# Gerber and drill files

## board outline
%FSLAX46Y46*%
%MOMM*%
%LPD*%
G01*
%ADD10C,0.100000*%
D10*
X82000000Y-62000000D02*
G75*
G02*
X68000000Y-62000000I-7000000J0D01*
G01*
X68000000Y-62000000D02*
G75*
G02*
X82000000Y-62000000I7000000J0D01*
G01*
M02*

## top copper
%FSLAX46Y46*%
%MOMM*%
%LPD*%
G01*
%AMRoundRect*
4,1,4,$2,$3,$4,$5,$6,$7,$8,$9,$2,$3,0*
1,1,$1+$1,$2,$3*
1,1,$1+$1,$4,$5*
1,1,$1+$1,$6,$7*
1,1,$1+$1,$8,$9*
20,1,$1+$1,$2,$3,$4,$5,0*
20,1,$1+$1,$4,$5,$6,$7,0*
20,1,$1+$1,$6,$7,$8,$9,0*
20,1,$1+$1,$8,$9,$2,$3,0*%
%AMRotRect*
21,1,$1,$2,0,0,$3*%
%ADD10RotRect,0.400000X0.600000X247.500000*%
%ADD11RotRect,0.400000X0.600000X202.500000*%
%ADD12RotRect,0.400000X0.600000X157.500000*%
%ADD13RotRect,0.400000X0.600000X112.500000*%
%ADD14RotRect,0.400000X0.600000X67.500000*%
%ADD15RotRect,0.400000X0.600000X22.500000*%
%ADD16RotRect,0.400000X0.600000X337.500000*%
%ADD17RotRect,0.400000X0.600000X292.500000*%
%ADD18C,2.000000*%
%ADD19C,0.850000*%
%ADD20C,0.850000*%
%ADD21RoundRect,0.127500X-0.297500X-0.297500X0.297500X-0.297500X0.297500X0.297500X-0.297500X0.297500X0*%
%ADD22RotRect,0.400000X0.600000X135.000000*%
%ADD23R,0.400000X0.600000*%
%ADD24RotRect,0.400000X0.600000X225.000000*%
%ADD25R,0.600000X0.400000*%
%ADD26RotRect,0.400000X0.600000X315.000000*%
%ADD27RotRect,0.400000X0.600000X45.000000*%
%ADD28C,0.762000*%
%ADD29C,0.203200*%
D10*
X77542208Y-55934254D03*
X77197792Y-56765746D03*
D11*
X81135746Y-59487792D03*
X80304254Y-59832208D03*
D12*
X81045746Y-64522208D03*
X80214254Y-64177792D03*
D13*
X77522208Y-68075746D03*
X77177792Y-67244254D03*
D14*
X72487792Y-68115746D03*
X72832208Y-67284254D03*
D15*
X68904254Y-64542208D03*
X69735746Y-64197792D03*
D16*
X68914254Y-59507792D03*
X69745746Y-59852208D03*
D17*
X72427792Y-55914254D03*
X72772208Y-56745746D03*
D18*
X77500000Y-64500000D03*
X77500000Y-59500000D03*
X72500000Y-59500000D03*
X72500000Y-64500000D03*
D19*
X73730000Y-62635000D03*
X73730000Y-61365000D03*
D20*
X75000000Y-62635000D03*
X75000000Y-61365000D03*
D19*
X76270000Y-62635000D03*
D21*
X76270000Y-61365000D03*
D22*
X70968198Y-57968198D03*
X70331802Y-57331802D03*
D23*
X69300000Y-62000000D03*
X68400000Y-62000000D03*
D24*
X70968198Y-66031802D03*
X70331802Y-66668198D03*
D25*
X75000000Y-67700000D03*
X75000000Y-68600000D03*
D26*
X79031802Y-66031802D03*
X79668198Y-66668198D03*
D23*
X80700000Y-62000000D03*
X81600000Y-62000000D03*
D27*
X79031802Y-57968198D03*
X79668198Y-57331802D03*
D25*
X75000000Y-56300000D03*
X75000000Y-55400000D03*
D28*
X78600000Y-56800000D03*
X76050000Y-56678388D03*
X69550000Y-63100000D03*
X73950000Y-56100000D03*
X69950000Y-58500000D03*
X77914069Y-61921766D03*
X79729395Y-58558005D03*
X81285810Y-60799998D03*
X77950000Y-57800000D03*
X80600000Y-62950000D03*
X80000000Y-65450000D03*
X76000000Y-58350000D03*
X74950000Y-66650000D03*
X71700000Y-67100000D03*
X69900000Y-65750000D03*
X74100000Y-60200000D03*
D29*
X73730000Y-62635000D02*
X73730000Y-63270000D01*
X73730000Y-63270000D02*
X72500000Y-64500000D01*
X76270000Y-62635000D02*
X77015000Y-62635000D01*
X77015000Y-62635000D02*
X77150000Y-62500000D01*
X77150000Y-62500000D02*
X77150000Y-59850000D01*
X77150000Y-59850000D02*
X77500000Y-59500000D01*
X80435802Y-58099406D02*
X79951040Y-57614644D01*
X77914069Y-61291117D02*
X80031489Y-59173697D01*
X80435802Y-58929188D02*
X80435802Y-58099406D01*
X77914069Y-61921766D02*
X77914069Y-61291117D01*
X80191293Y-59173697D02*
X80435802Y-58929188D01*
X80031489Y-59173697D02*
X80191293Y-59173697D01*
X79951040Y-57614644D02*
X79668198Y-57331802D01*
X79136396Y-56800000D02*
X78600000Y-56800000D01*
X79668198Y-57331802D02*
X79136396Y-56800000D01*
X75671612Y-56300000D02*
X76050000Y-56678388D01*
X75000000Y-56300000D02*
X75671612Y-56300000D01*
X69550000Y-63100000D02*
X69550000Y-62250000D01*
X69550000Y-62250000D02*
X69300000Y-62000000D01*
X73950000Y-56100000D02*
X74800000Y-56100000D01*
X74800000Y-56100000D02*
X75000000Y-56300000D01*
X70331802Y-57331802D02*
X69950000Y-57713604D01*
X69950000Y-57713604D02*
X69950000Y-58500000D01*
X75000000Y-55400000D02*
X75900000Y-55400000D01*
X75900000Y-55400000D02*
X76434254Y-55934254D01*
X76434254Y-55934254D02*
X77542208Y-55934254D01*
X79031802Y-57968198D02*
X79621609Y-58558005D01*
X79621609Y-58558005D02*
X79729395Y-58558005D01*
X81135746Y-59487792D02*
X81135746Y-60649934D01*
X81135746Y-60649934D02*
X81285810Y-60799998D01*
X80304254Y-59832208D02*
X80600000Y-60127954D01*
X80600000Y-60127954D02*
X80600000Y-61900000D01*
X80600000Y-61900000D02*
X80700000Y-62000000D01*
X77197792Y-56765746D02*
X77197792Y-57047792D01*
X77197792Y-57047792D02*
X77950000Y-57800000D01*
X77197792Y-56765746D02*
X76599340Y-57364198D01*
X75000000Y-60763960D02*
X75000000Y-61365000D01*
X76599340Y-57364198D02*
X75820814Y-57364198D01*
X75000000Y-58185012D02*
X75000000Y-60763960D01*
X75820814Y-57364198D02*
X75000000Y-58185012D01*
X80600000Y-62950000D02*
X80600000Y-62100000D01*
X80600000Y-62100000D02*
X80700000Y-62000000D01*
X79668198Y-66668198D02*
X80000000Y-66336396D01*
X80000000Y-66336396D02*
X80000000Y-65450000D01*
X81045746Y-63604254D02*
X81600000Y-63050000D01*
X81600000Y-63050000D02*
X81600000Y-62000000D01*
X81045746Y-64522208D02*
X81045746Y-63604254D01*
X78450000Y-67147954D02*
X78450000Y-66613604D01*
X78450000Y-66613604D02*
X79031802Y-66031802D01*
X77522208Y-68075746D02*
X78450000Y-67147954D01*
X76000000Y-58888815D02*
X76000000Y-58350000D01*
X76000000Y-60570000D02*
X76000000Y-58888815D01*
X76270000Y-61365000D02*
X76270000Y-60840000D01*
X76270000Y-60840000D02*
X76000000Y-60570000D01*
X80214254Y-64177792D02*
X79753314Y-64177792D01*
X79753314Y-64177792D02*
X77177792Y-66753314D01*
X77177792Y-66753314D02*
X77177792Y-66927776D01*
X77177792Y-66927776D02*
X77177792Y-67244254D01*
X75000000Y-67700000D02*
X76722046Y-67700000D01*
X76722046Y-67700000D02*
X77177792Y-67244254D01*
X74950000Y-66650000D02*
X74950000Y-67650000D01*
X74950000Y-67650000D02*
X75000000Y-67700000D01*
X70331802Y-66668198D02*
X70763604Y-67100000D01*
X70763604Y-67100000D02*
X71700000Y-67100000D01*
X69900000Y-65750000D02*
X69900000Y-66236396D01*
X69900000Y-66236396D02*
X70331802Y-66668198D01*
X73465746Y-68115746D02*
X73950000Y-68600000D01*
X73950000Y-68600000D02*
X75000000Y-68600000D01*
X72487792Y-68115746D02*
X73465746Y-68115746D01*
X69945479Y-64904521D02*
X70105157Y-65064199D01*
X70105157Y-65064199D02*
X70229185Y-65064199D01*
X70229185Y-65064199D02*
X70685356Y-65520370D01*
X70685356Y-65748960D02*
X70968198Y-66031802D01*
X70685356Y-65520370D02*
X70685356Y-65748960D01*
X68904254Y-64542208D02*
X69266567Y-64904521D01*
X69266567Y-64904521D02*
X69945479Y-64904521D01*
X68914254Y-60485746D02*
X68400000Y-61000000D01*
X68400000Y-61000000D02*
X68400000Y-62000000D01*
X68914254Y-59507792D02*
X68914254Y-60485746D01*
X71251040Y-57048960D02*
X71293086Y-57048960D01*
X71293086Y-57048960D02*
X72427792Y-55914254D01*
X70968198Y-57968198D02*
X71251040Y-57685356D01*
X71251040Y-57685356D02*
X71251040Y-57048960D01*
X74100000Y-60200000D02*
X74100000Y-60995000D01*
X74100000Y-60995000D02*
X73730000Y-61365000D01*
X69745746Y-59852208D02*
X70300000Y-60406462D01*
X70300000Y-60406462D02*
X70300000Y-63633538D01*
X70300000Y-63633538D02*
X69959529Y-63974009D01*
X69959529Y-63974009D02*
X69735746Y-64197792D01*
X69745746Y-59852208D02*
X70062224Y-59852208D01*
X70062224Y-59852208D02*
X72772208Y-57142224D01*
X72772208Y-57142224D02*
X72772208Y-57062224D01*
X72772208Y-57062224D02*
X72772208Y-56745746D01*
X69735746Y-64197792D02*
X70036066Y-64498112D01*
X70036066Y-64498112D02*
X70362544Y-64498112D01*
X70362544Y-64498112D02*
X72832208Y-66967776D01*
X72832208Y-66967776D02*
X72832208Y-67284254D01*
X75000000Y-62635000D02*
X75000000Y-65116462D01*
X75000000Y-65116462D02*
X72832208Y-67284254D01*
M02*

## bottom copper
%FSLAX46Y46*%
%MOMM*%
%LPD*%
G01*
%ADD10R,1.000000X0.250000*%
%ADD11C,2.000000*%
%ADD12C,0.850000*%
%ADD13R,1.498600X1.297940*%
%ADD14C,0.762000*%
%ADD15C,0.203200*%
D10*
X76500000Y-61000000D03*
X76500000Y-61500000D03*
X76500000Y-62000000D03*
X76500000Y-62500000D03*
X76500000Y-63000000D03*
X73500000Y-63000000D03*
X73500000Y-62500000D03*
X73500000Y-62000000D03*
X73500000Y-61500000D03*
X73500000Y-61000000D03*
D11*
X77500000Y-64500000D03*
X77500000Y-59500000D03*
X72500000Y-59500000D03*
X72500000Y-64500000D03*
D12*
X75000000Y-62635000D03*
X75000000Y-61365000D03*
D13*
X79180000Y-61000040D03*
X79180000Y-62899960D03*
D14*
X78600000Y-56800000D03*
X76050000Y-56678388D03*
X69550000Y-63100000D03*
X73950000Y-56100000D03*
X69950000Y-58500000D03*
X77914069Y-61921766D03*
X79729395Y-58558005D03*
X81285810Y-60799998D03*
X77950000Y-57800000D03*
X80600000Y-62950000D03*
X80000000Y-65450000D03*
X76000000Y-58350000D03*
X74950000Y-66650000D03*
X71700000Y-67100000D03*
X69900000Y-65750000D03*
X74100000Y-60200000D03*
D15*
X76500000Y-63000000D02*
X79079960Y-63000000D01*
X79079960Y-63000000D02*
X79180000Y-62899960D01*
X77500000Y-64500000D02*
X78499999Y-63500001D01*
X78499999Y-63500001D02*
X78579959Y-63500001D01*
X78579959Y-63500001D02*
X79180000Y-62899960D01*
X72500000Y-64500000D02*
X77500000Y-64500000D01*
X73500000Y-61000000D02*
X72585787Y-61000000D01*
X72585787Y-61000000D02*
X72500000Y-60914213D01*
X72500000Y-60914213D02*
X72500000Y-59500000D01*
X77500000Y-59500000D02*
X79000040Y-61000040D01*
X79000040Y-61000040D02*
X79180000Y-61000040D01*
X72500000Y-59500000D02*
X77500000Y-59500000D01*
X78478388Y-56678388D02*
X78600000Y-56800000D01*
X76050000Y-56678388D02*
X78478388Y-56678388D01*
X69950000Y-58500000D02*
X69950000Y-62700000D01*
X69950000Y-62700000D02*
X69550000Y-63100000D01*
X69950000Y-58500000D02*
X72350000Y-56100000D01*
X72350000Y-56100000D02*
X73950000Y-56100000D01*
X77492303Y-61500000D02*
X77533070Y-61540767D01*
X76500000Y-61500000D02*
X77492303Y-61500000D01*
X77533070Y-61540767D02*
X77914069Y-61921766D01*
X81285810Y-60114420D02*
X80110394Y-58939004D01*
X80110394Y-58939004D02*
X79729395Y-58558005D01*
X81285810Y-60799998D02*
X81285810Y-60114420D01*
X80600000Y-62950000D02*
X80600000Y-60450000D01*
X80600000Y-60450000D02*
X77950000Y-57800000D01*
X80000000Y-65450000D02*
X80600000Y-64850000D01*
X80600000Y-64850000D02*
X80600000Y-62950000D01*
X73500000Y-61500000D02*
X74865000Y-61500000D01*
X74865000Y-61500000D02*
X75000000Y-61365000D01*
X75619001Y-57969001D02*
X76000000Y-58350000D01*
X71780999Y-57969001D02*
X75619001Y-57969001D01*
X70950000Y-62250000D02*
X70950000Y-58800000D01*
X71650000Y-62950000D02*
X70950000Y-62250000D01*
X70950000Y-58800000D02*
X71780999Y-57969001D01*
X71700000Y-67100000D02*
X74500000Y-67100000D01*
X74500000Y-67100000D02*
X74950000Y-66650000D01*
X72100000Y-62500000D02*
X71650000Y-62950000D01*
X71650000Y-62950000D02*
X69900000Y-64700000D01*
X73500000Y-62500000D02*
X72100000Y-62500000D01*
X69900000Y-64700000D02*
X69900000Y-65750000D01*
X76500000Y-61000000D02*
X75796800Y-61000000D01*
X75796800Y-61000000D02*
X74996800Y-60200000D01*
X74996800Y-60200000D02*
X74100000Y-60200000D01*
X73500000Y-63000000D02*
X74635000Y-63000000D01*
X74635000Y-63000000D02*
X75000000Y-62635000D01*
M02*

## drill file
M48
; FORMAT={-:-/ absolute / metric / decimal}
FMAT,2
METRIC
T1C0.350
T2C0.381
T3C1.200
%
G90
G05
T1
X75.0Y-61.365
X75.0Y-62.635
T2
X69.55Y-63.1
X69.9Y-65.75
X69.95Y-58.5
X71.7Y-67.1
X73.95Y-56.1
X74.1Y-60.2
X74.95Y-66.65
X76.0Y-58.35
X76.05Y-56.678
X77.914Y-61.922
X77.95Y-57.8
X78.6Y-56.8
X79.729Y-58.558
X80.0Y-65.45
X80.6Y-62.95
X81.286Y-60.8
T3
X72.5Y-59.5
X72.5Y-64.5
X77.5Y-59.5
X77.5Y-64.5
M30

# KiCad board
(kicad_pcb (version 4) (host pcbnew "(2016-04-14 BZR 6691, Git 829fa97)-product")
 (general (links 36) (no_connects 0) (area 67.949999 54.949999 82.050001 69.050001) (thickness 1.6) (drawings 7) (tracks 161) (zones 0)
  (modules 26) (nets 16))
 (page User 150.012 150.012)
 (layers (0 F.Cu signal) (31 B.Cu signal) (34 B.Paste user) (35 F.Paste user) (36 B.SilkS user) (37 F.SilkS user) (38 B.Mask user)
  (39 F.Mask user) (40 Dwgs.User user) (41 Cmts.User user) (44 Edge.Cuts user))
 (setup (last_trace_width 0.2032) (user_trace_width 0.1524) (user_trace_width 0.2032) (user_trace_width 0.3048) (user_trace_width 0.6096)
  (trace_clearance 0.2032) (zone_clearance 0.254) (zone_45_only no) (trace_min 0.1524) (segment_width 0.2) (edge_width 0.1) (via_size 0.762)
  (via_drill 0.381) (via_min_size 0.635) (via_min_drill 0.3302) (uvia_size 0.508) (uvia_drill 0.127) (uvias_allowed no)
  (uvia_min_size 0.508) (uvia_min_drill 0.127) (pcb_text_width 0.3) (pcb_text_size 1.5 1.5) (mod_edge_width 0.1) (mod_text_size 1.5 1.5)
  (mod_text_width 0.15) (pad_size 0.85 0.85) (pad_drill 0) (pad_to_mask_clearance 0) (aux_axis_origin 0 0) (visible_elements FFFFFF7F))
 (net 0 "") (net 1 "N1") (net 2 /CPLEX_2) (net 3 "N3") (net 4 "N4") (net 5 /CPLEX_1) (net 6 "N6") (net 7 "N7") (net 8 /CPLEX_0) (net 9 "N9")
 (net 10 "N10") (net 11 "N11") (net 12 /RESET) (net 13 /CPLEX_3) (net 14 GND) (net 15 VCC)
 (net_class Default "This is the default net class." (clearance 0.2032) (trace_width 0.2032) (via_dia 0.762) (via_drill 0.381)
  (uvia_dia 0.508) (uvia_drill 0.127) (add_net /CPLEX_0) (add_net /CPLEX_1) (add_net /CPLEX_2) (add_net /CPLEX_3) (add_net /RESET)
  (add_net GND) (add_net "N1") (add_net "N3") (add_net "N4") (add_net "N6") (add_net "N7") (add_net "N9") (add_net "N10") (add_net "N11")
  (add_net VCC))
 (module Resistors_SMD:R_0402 (layer F.Cu) (at 77.37 56.35 247.5)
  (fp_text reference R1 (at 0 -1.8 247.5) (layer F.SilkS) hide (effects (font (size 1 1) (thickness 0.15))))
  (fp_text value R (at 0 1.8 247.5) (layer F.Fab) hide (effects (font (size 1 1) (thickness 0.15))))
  (pad 1 smd rect (at -0.45 0 247.5) (size 0.4 0.6) (layers F.Cu F.Paste F.Mask) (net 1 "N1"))
  (pad 2 smd rect (at 0.45 0 247.5) (size 0.4 0.6) (layers F.Cu F.Paste F.Mask) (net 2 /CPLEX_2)))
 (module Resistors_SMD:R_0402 (layer F.Cu) (at 80.72 59.66 202.5)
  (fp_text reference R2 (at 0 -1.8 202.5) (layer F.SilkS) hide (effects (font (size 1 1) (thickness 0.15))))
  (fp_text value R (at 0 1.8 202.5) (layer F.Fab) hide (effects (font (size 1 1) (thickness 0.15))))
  (pad 1 smd rect (at -0.45 0 202.5) (size 0.4 0.6) (layers F.Cu F.Paste F.Mask) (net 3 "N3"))
  (pad 2 smd rect (at 0.45 0 202.5) (size 0.4 0.6) (layers F.Cu F.Paste F.Mask) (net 2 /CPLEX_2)))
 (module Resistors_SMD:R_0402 (layer F.Cu) (at 80.63 64.35 157.5)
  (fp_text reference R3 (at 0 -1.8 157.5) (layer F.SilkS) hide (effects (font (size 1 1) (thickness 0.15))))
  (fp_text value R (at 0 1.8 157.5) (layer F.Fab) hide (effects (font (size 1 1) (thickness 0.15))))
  (pad 1 smd rect (at -0.45 0 157.5) (size 0.4 0.6) (layers F.Cu F.Paste F.Mask) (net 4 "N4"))
  (pad 2 smd rect (at 0.45 0 157.5) (size 0.4 0.6) (layers F.Cu F.Paste F.Mask) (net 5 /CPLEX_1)))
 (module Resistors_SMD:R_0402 (layer F.Cu) (at 77.35 67.66 112.5)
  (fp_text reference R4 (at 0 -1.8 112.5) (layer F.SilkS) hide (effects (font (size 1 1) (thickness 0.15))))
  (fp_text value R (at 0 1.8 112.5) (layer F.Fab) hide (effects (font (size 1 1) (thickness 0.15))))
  (pad 1 smd rect (at -0.45 0 112.5) (size 0.4 0.6) (layers F.Cu F.Paste F.Mask) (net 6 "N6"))
  (pad 2 smd rect (at 0.45 0 112.5) (size 0.4 0.6) (layers F.Cu F.Paste F.Mask) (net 5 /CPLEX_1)))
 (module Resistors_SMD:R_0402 (layer F.Cu) (at 72.66 67.7 67.5)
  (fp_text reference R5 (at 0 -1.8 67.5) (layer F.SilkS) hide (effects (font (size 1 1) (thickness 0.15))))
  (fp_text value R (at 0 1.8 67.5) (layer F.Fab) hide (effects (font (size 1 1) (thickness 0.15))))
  (pad 1 smd rect (at -0.45 0 67.5) (size 0.4 0.6) (layers F.Cu F.Paste F.Mask) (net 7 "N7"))
  (pad 2 smd rect (at 0.45 0 67.5) (size 0.4 0.6) (layers F.Cu F.Paste F.Mask) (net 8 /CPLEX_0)))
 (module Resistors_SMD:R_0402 (layer F.Cu) (at 69.32 64.37 22.5)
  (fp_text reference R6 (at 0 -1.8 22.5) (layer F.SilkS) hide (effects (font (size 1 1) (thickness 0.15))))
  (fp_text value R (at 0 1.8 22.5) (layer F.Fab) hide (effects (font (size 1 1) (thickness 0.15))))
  (pad 1 smd rect (at -0.45 0 22.5) (size 0.4 0.6) (layers F.Cu F.Paste F.Mask) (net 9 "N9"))
  (pad 2 smd rect (at 0.45 0 22.5) (size 0.4 0.6) (layers F.Cu F.Paste F.Mask) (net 8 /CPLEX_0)))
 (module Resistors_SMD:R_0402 (layer F.Cu) (at 69.33 59.68 337.5)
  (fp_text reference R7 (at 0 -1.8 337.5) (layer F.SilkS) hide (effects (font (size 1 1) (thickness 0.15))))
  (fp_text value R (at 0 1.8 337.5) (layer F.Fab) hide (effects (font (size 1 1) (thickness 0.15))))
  (pad 1 smd rect (at -0.45 0 337.5) (size 0.4 0.6) (layers F.Cu F.Paste F.Mask) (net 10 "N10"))
  (pad 2 smd rect (at 0.45 0 337.5) (size 0.4 0.6) (layers F.Cu F.Paste F.Mask) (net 8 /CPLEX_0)))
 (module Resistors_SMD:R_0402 (layer F.Cu) (at 72.6 56.33 292.5)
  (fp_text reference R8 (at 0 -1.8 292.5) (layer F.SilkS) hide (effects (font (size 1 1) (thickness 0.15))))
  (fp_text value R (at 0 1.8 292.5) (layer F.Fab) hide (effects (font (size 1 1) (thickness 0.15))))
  (pad 1 smd rect (at -0.45 0 292.5) (size 0.4 0.6) (layers F.Cu F.Paste F.Mask) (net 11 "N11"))
  (pad 2 smd rect (at 0.45 0 292.5) (size 0.4 0.6) (layers F.Cu F.Paste F.Mask) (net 8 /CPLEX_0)))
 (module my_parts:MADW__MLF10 (layer B.Cu) (at 75 62 180)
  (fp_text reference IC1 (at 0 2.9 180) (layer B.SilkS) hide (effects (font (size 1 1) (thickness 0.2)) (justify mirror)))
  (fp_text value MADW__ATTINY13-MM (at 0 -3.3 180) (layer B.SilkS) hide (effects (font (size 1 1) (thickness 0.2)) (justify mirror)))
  (pad 1 smd rect (at -1.5 1 180) (size 1 0.25) (layers B.Cu B.Paste B.Mask) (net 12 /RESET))
  (pad 2 smd rect (at -1.5 0.5 180) (size 1 0.25) (layers B.Cu B.Paste B.Mask) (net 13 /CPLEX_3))
  (pad 3 smd rect (at -1.5 0 180) (size 1 0.25) (layers B.Cu B.Paste B.Mask))
  (pad 4 smd rect (at -1.5 -0.5 180) (size 1 0.25) (layers B.Cu B.Paste B.Mask))
  (pad 5 smd rect (at -1.5 -1 180) (size 1 0.25) (layers B.Cu B.Paste B.Mask) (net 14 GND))
  (pad 6 smd rect (at 1.5 -1 180) (size 1 0.25) (layers B.Cu B.Paste B.Mask) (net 8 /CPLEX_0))
  (pad 7 smd rect (at 1.5 -0.5 180) (size 1 0.25) (layers B.Cu B.Paste B.Mask) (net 5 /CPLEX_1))
  (pad 8 smd rect (at 1.5 0 180) (size 1 0.25) (layers B.Cu B.Paste B.Mask))
  (pad 9 smd rect (at 1.5 0.5 180) (size 1 0.25) (layers B.Cu B.Paste B.Mask) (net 2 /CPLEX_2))
  (pad 10 smd rect (at 1.5 1 180) (size 1 0.25) (layers B.Cu B.Paste B.Mask) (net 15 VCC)))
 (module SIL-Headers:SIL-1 (layer F.Cu) (at 77.5 64.5)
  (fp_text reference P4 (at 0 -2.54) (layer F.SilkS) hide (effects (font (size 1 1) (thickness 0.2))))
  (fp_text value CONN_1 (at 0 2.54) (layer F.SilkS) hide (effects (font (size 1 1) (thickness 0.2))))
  (pad 1 thru_hole circle (at 0 0) (size 2 2) (drill 1.2) (layers *.Cu *.Mask) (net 14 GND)))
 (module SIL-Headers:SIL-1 (layer F.Cu) (at 77.5 59.5)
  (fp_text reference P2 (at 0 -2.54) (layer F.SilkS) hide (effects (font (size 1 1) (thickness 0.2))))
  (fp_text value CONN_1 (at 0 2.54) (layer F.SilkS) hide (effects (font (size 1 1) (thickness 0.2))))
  (pad 1 thru_hole circle (at 0 0) (size 2 2) (drill 1.2) (layers *.Cu *.Mask) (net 15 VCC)))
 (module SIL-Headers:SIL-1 (layer F.Cu) (at 72.5 59.5)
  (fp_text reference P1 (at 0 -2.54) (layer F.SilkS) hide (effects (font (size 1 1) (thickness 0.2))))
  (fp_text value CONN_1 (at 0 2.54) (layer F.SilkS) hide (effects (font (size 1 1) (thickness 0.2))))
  (pad 1 thru_hole circle (at 0 0) (size 2 2) (drill 1.2) (layers *.Cu *.Mask) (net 15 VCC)))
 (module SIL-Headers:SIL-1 (layer F.Cu) (at 72.5 64.5)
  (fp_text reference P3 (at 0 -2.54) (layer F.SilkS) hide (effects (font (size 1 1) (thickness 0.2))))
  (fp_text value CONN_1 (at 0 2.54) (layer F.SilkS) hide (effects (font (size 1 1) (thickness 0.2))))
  (pad 1 thru_hole circle (at 0 0) (size 2 2) (drill 1.2) (layers *.Cu *.Mask) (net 14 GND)))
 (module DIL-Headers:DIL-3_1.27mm (layer F.Cu) (at 75 62) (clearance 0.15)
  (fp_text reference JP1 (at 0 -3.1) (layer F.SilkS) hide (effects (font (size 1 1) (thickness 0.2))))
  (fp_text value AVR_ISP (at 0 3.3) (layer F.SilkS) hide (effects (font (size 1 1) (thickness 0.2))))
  (pad 6 smd circle (at -1.27 0.635) (size 0.85 0.85) (layers F.Cu F.Mask) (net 14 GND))
  (pad 5 smd circle (at -1.27 -0.635) (size 0.85 0.85) (layers F.Cu F.Mask) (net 12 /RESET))
  (pad 4 thru_hole circle (at 0 0.635) (size 0.85 0.85) (drill 0.35) (layers *.Cu F.Mask) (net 8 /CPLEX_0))
  (pad 3 thru_hole circle (at 0 -0.635) (size 0.85 0.85) (drill 0.35) (layers *.Cu F.Mask) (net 2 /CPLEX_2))
  (pad 2 smd circle (at 1.27 0.635) (size 0.85 0.85) (layers F.Cu F.Mask) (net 15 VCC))
  (pad 1 smd roundrect (at 1.27 -0.635) (size 0.85 0.85) (layers F.Cu F.Mask) (roundrect_rratio 0.15) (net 5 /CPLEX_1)))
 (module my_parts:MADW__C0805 (layer B.Cu) (at 79.18 61.95 270)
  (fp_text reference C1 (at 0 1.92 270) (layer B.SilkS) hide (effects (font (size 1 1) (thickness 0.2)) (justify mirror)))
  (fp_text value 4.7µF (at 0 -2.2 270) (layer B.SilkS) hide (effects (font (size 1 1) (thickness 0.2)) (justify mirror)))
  (pad 1 smd rect (at -0.94996 0 270) (size 1.29794 1.4986) (layers B.Cu B.Paste B.Mask) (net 15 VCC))
  (pad 2 smd rect (at 0.94996 0 270) (size 1.29794 1.4986) (layers B.Cu B.Paste B.Mask) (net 14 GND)))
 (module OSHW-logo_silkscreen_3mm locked (layer B.Cu) (at 75 56.8)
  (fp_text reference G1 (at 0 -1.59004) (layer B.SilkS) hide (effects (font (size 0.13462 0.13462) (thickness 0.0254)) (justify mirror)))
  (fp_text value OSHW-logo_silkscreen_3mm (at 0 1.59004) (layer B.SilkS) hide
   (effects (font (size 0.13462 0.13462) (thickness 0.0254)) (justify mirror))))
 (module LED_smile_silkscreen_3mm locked (layer B.Cu) (at 75 67.2)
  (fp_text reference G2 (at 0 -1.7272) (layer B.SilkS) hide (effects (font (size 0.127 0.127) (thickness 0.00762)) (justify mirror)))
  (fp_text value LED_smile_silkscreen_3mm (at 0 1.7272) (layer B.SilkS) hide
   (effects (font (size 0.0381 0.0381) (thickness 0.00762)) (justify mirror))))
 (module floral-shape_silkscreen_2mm (layer F.Cu) (at 75.03 57.9 45)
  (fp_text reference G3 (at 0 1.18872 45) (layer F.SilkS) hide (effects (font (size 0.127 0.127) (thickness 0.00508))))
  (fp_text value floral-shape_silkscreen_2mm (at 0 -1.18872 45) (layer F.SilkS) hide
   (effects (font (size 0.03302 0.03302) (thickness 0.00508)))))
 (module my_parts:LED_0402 (layer F.Cu) (at 70.65 57.65 135)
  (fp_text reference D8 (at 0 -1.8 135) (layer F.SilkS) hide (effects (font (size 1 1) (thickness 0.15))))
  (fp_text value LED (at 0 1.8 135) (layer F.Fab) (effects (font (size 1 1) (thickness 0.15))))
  (pad 1 smd rect (at -0.45 0 135) (size 0.4 0.6) (layers F.Cu F.Paste F.Mask) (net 11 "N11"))
  (pad 2 smd rect (at 0.45 0 135) (size 0.4 0.6) (layers F.Cu F.Paste F.Mask) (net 13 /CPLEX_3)))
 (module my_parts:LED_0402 (layer F.Cu) (at 68.85 62 180)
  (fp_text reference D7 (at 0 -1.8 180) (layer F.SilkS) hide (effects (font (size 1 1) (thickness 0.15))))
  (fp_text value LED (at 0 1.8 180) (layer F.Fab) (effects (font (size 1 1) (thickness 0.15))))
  (pad 1 smd rect (at -0.45 0 180) (size 0.4 0.6) (layers F.Cu F.Paste F.Mask) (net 13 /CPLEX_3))
  (pad 2 smd rect (at 0.45 0 180) (size 0.4 0.6) (layers F.Cu F.Paste F.Mask) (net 10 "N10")))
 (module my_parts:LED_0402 (layer F.Cu) (at 70.65 66.35 225)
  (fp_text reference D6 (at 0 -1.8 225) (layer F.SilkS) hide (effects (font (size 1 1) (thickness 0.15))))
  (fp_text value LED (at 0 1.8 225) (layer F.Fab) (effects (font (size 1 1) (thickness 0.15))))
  (pad 1 smd rect (at -0.45 0 225) (size 0.4 0.6) (layers F.Cu F.Paste F.Mask) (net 9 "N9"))
  (pad 2 smd rect (at 0.45 0 225) (size 0.4 0.6) (layers F.Cu F.Paste F.Mask) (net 5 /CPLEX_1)))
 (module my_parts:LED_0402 (layer F.Cu) (at 75 68.15 270)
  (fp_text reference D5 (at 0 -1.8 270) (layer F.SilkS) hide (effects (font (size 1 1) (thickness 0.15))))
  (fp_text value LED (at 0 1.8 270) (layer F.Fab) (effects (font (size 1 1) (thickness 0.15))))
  (pad 1 smd rect (at -0.45 0 270) (size 0.4 0.6) (layers F.Cu F.Paste F.Mask) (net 5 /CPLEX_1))
  (pad 2 smd rect (at 0.45 0 270) (size 0.4 0.6) (layers F.Cu F.Paste F.Mask) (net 7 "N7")))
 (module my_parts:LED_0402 (layer F.Cu) (at 79.35 66.35 315)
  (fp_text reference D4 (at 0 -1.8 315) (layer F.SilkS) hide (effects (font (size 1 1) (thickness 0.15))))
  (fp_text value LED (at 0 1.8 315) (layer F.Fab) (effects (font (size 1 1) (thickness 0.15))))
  (pad 1 smd rect (at -0.45 0 315) (size 0.4 0.6) (layers F.Cu F.Paste F.Mask) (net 6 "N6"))
  (pad 2 smd rect (at 0.45 0 315) (size 0.4 0.6) (layers F.Cu F.Paste F.Mask) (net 2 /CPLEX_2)))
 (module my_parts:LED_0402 (layer F.Cu) (at 81.15 62)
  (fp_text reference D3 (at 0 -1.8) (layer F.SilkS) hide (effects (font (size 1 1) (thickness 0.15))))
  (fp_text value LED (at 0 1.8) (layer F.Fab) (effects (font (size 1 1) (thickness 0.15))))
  (pad 1 smd rect (at -0.45 0) (size 0.4 0.6) (layers F.Cu F.Paste F.Mask) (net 2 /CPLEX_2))
  (pad 2 smd rect (at 0.45 0) (size 0.4 0.6) (layers F.Cu F.Paste F.Mask) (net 4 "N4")))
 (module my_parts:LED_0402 (layer F.Cu) (at 79.35 57.65 45)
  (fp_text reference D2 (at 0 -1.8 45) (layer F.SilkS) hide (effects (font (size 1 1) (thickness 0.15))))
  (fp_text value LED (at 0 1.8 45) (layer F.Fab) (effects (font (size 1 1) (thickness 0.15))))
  (pad 1 smd rect (at -0.45 0 45) (size 0.4 0.6) (layers F.Cu F.Paste F.Mask) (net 3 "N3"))
  (pad 2 smd rect (at 0.45 0 45) (size 0.4 0.6) (layers F.Cu F.Paste F.Mask) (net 13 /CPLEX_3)))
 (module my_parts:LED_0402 (layer F.Cu) (at 75 55.85 90)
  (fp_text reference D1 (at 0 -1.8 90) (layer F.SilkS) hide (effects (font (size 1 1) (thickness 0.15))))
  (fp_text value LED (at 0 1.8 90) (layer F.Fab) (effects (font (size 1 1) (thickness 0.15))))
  (pad 1 smd rect (at -0.45 0 90) (size 0.4 0.6) (layers F.Cu F.Paste F.Mask) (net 13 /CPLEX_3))
  (pad 2 smd rect (at 0.45 0 90) (size 0.4 0.6) (layers F.Cu F.Paste F.Mask) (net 1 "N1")))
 (gr_circle (center 75 62) (end 82 62) (layer Edge.Cuts) (width 0.1))
 (segment (start 73.73 62.635) (end 73.73 63.27) (width 0.2032) (layer F.Cu) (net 14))
 (segment (start 73.73 63.27) (end 72.5 64.5) (width 0.2032) (layer F.Cu) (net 14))
 (segment (start 76.5 63) (end 79.07996 63) (width 0.2032) (layer B.Cu) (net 14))
 (segment (start 79.07996 63) (end 79.18 62.89996) (width 0.2032) (layer B.Cu) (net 14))
 (segment (start 77.5 64.5) (end 78.499999 63.500001) (width 0.2032) (layer B.Cu) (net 14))
 (segment (start 78.499999 63.500001) (end 78.579959 63.500001) (width 0.2032) (layer B.Cu) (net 14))
 (segment (start 78.579959 63.500001) (end 79.18 62.89996) (width 0.2032) (layer B.Cu) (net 14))
 (segment (start 72.5 64.5) (end 77.5 64.5) (width 0.2032) (layer B.Cu) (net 14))
 (segment (start 76.27 62.635) (end 77.015 62.635) (width 0.2032) (layer F.Cu) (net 15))
 (segment (start 77.015 62.635) (end 77.15 62.5) (width 0.2032) (layer F.Cu) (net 15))
 (segment (start 77.15 62.5) (end 77.15 59.85) (width 0.2032) (layer F.Cu) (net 15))
 (segment (start 77.15 59.85) (end 77.5 59.5) (width 0.2032) (layer F.Cu) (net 15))
 (segment (start 73.5 61) (end 72.585787 61) (width 0.2032) (layer B.Cu) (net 15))
 (segment (start 72.585787 61) (end 72.5 60.914213) (width 0.2032) (layer B.Cu) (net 15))
 (segment (start 72.5 60.914213) (end 72.5 59.5) (width 0.2032) (layer B.Cu) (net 15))
 (segment (start 77.5 59.5) (end 79.00004 61.00004) (width 0.2032) (layer B.Cu) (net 15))
 (segment (start 79.00004 61.00004) (end 79.18 61.00004) (width 0.2032) (layer B.Cu) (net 15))
 (segment (start 72.5 59.5) (end 77.5 59.5) (width 0.2032) (layer B.Cu) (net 15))
 (segment (start 80.435802 58.099406) (end 79.95104 57.614644) (width 0.2032) (layer F.Cu) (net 13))
 (segment (start 77.914069 61.291117) (end 80.031489 59.173697) (width 0.2032) (layer F.Cu) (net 13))
 (segment (start 80.435802 58.929188) (end 80.435802 58.099406) (width 0.2032) (layer F.Cu) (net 13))
 (segment (start 77.914069 61.921766) (end 77.914069 61.291117) (width 0.2032) (layer F.Cu) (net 13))
 (segment (start 80.191293 59.173697) (end 80.435802 58.929188) (width 0.2032) (layer F.Cu) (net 13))
 (segment (start 80.031489 59.173697) (end 80.191293 59.173697) (width 0.2032) (layer F.Cu) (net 13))
 (segment (start 79.95104 57.614644) (end 79.668198 57.331802) (width 0.2032) (layer F.Cu) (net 13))
 (segment (start 79.136396 56.8) (end 78.6 56.8) (width 0.2032) (layer F.Cu) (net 13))
 (segment (start 79.668198 57.331802) (end 79.136396 56.8) (width 0.2032) (layer F.Cu) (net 13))
 (segment (start 78.478388 56.678388) (end 78.6 56.8) (width 0.2032) (layer B.Cu) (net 13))
 (segment (start 76.05 56.678388) (end 78.478388 56.678388) (width 0.2032) (layer B.Cu) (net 13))
 (via (at 78.6 56.8) (size 0.762) (drill 0.381) (layers F.Cu B.Cu) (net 13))
 (segment (start 75.671612 56.3) (end 76.05 56.678388) (width 0.2032) (layer F.Cu) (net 13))
 (via (at 76.05 56.678388) (size 0.762) (drill 0.381) (layers F.Cu B.Cu) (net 13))
 (segment (start 75 56.3) (end 75.671612 56.3) (width 0.2032) (layer F.Cu) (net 13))
 (segment (start 69.55 63.1) (end 69.55 62.25) (width 0.2032) (layer F.Cu) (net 13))
 (segment (start 69.55 62.25) (end 69.3 62) (width 0.2032) (layer F.Cu) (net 13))
 (segment (start 69.95 58.5) (end 69.95 62.7) (width 0.2032) (layer B.Cu) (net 13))
 (segment (start 69.95 62.7) (end 69.55 63.1) (width 0.2032) (layer B.Cu) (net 13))
 (via (at 69.55 63.1) (size 0.762) (drill 0.381) (layers F.Cu B.Cu) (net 13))
 (segment (start 73.95 56.1) (end 74.8 56.1) (width 0.2032) (layer F.Cu) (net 13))
 (segment (start 74.8 56.1) (end 75 56.3) (width 0.2032) (layer F.Cu) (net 13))
 (segment (start 69.95 58.5) (end 72.35 56.1) (width 0.2032) (layer B.Cu) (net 13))
 (segment (start 72.35 56.1) (end 73.95 56.1) (width 0.2032) (layer B.Cu) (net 13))
 (via (at 73.95 56.1) (size 0.762) (drill 0.381) (layers F.Cu B.Cu) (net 13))
 (segment (start 70.331802 57.331802) (end 69.95 57.713604) (width 0.2032) (layer F.Cu) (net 13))
 (segment (start 69.95 57.713604) (end 69.95 58.5) (width 0.2032) (layer F.Cu) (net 13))
 (via (at 69.95 58.5) (size 0.762) (drill 0.381) (layers F.Cu B.Cu) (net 13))
 (segment (start 77.492303 61.5) (end 77.53307 61.540767) (width 0.2032) (layer B.Cu) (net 13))
 (segment (start 76.5 61.5) (end 77.492303 61.5) (width 0.2032) (layer B.Cu) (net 13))
 (segment (start 77.53307 61.540767) (end 77.914069 61.921766) (width 0.2032) (layer B.Cu) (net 13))
 (via (at 77.914069 61.921766) (size 0.762) (drill 0.381) (layers F.Cu B.Cu) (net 13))
 (segment (start 75 55.4) (end 75.9 55.4) (width 0.2032) (layer F.Cu) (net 1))
 (segment (start 75.9 55.4) (end 76.434254 55.934254) (width 0.2032) (layer F.Cu) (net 1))
 (segment (start 76.434254 55.934254) (end 77.542208 55.934254) (width 0.2032) (layer F.Cu) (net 1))
 (segment (start 81.28581 60.11442) (end 80.110394 58.939004) (width 0.2032) (layer B.Cu) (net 3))
 (segment (start 80.110394 58.939004) (end 79.729395 58.558005) (width 0.2032) (layer B.Cu) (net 3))
 (segment (start 81.28581 60.799998) (end 81.28581 60.11442) (width 0.2032) (layer B.Cu) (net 3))
 (segment (start 79.031802 57.968198) (end 79.621609 58.558005) (width 0.2032) (layer F.Cu) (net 3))
 (segment (start 79.621609 58.558005) (end 79.729395 58.558005) (width 0.2032) (layer F.Cu) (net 3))
 (via (at 79.729395 58.558005) (size 0.762) (drill 0.381) (layers F.Cu B.Cu) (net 3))
 (segment (start 81.135746 59.487792) (end 81.135746 60.649934) (width 0.2032) (layer F.Cu) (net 3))
 (via (at 81.28581 60.799998) (size 0.762) (drill 0.381) (layers F.Cu B.Cu) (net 3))
 (segment (start 81.135746 60.649934) (end 81.28581 60.799998) (width 0.2032) (layer F.Cu) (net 3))
 (segment (start 80.6 62.95) (end 80.6 60.45) (width 0.2032) (layer B.Cu) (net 2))
 (segment (start 80.6 60.45) (end 77.95 57.8) (width 0.2032) (layer B.Cu) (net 2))
 (segment (start 80.304254 59.832208) (end 80.6 60.127954) (width 0.2032) (layer F.Cu) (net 2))
 (segment (start 80.6 60.127954) (end 80.6 61.9) (width 0.2032) (layer F.Cu) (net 2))
 (segment (start 80.6 61.9) (end 80.7 62) (width 0.2032) (layer F.Cu) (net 2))
 (segment (start 77.197792 56.765746) (end 77.197792 57.047792) (width 0.2032) (layer F.Cu) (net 2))
 (segment (start 77.197792 57.047792) (end 77.95 57.8) (width 0.2032) (layer F.Cu) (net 2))
 (via (at 77.95 57.8) (size 0.762) (drill 0.381) (layers F.Cu B.Cu) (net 2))
 (segment (start 77.197792 56.765746) (end 76.59934 57.364198) (width 0.2032) (layer F.Cu) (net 2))
 (segment (start 75 60.76396) (end 75 61.365) (width 0.2032) (layer F.Cu) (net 2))
 (segment (start 76.59934 57.364198) (end 75.820814 57.364198) (width 0.2032) (layer F.Cu) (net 2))
 (segment (start 75 58.185012) (end 75 60.76396) (width 0.2032) (layer F.Cu) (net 2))
 (segment (start 75.820814 57.364198) (end 75 58.185012) (width 0.2032) (layer F.Cu) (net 2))
 (segment (start 80.6 62.95) (end 80.6 62.1) (width 0.2032) (layer F.Cu) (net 2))
 (segment (start 80.6 62.1) (end 80.7 62) (width 0.2032) (layer F.Cu) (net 2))
 (segment (start 80 65.45) (end 80.6 64.85) (width 0.2032) (layer B.Cu) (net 2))
 (via (at 80.6 62.95) (size 0.762) (drill 0.381) (layers F.Cu B.Cu) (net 2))
 (segment (start 80.6 64.85) (end 80.6 62.95) (width 0.2032) (layer B.Cu) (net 2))
 (segment (start 79.668198 66.668198) (end 80 66.336396) (width 0.2032) (layer F.Cu) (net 2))
 (segment (start 80 66.336396) (end 80 65.45) (width 0.2032) (layer F.Cu) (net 2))
 (via (at 80 65.45) (size 0.762) (drill 0.381) (layers F.Cu B.Cu) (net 2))
 (segment (start 73.5 61.5) (end 74.865 61.5) (width 0.2032) (layer B.Cu) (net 2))
 (segment (start 74.865 61.5) (end 75 61.365) (width 0.2032) (layer B.Cu) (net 2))
 (segment (start 81.045746 63.604254) (end 81.6 63.05) (width 0.2032) (layer F.Cu) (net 4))
 (segment (start 81.6 63.05) (end 81.6 62) (width 0.2032) (layer F.Cu) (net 4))
 (segment (start 81.045746 64.522208) (end 81.045746 63.604254) (width 0.2032) (layer F.Cu) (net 4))
 (segment (start 78.45 67.147954) (end 78.45 66.613604) (width 0.2032) (layer F.Cu) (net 6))
 (segment (start 78.45 66.613604) (end 79.031802 66.031802) (width 0.2032) (layer F.Cu) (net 6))
 (segment (start 77.522208 68.075746) (end 78.45 67.147954) (width 0.2032) (layer F.Cu) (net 6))
 (segment (start 75.619001 57.969001) (end 76 58.35) (width 0.2032) (layer B.Cu) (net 5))
 (segment (start 71.780999 57.969001) (end 75.619001 57.969001) (width 0.2032) (layer B.Cu) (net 5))
 (segment (start 70.95 62.25) (end 70.95 58.8) (width 0.2032) (layer B.Cu) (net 5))
 (segment (start 76 58.888815) (end 76 58.35) (width 0.2032) (layer F.Cu) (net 5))
 (segment (start 76 60.57) (end 76 58.888815) (width 0.2032) (layer F.Cu) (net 5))
 (segment (start 76.27 61.365) (end 76.27 60.84) (width 0.2032) (layer F.Cu) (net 5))
 (segment (start 71.65 62.95) (end 70.95 62.25) (width 0.2032) (layer B.Cu) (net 5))
 (segment (start 70.95 58.8) (end 71.780999 57.969001) (width 0.2032) (layer B.Cu) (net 5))
 (segment (start 76.27 60.84) (end 76 60.57) (width 0.2032) (layer F.Cu) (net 5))
 (via (at 76 58.35) (size 0.762) (drill 0.381) (layers F.Cu B.Cu) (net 5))
 (segment (start 80.214254 64.177792) (end 79.753314 64.177792) (width 0.2032) (layer F.Cu) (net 5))
 (segment (start 79.753314 64.177792) (end 77.177792 66.753314) (width 0.2032) (layer F.Cu) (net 5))
 (segment (start 77.177792 66.753314) (end 77.177792 66.927776) (width 0.2032) (layer F.Cu) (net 5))
 (segment (start 77.177792 66.927776) (end 77.177792 67.244254) (width 0.2032) (layer F.Cu) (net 5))
 (segment (start 75 67.7) (end 76.722046 67.7) (width 0.2032) (layer F.Cu) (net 5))
 (segment (start 76.722046 67.7) (end 77.177792 67.244254) (width 0.2032) (layer F.Cu) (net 5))
 (segment (start 74.95 66.65) (end 74.95 67.65) (width 0.2032) (layer F.Cu) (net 5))
 (segment (start 74.95 67.65) (end 75 67.7) (width 0.2032) (layer F.Cu) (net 5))
 (segment (start 71.7 67.1) (end 74.5 67.1) (width 0.2032) (layer B.Cu) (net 5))
 (via (at 74.95 66.65) (size 0.762) (drill 0.381) (layers F.Cu B.Cu) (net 5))
 (segment (start 74.5 67.1) (end 74.95 66.65) (width 0.2032) (layer B.Cu) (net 5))
 (segment (start 70.331802 66.668198) (end 70.763604 67.1) (width 0.2032) (layer F.Cu) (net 5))
 (segment (start 70.763604 67.1) (end 71.7 67.1) (width 0.2032) (layer F.Cu) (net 5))
 (via (at 71.7 67.1) (size 0.762) (drill 0.381) (layers F.Cu B.Cu) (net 5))
 (segment (start 72.1 62.5) (end 71.65 62.95) (width 0.2032) (layer B.Cu) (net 5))
 (segment (start 71.65 62.95) (end 69.9 64.7) (width 0.2032) (layer B.Cu) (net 5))
 (segment (start 73.5 62.5) (end 72.1 62.5) (width 0.2032) (layer B.Cu) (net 5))
 (segment (start 69.9 64.7) (end 69.9 65.75) (width 0.2032) (layer B.Cu) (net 5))
 (segment (start 69.9 65.75) (end 69.9 66.236396) (width 0.2032) (layer F.Cu) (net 5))
 (segment (start 69.9 66.236396) (end 70.331802 66.668198) (width 0.2032) (layer F.Cu) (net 5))
 (via (at 69.9 65.75) (size 0.762) (drill 0.381) (layers F.Cu B.Cu) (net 5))
 (segment (start 73.465746 68.115746) (end 73.95 68.6) (width 0.2032) (layer F.Cu) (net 7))
 (segment (start 73.95 68.6) (end 75 68.6) (width 0.2032) (layer F.Cu) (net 7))
 (segment (start 72.487792 68.115746) (end 73.465746 68.115746) (width 0.2032) (layer F.Cu) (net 7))
 (segment (start 69.945479 64.904521) (end 70.105157 65.064199) (width 0.2032) (layer F.Cu) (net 9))
 (segment (start 70.105157 65.064199) (end 70.229185 65.064199) (width 0.2032) (layer F.Cu) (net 9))
 (segment (start 70.229185 65.064199) (end 70.685356 65.52037) (width 0.2032) (layer F.Cu) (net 9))
 (segment (start 70.685356 65.74896) (end 70.968198 66.031802) (width 0.2032) (layer F.Cu) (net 9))
 (segment (start 70.685356 65.52037) (end 70.685356 65.74896) (width 0.2032) (layer F.Cu) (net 9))
 (segment (start 68.904254 64.542208) (end 69.266567 64.904521) (width 0.2032) (layer F.Cu) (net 9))
 (segment (start 69.266567 64.904521) (end 69.945479 64.904521) (width 0.2032) (layer F.Cu) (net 9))
 (segment (start 68.914254 60.485746) (end 68.4 61) (width 0.2032) (layer F.Cu) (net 10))
 (segment (start 68.4 61) (end 68.4 62) (width 0.2032) (layer F.Cu) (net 10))
 (segment (start 68.914254 59.507792) (end 68.914254 60.485746) (width 0.2032) (layer F.Cu) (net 10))
 (segment (start 71.25104 57.04896) (end 71.293086 57.04896) (width 0.2032) (layer F.Cu) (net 11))
 (segment (start 71.293086 57.04896) (end 72.427792 55.914254) (width 0.2032) (layer F.Cu) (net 11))
 (segment (start 70.968198 57.968198) (end 71.25104 57.685356) (width 0.2032) (layer F.Cu) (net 11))
 (segment (start 71.25104 57.685356) (end 71.25104 57.04896) (width 0.2032) (layer F.Cu) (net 11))
 (segment (start 74.1 60.2) (end 74.1 60.995) (width 0.2032) (layer F.Cu) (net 12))
 (segment (start 74.1 60.995) (end 73.73 61.365) (width 0.2032) (layer F.Cu) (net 12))
 (segment (start 76.5 61) (end 75.7968 61) (width 0.2032) (layer B.Cu) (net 12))
 (segment (start 75.7968 61) (end 74.9968 60.2) (width 0.2032) (layer B.Cu) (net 12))
 (segment (start 74.9968 60.2) (end 74.1 60.2) (width 0.2032) (layer B.Cu) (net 12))
 (via (at 74.1 60.2) (size 0.762) (drill 0.381) (layers F.Cu B.Cu) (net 12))
 (segment (start 69.745746 59.852208) (end 70.3 60.406462) (width 0.2032) (layer F.Cu) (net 8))
 (segment (start 70.3 60.406462) (end 70.3 63.633538) (width 0.2032) (layer F.Cu) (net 8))
 (segment (start 70.3 63.633538) (end 69.959529 63.974009) (width 0.2032) (layer F.Cu) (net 8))
 (segment (start 69.959529 63.974009) (end 69.735746 64.197792) (width 0.2032) (layer F.Cu) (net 8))
 (segment (start 69.745746 59.852208) (end 70.062224 59.852208) (width 0.2032) (layer F.Cu) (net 8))
 (segment (start 70.062224 59.852208) (end 72.772208 57.142224) (width 0.2032) (layer F.Cu) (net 8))
 (segment (start 72.772208 57.142224) (end 72.772208 57.062224) (width 0.2032) (layer F.Cu) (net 8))
 (segment (start 72.772208 57.062224) (end 72.772208 56.745746) (width 0.2032) (layer F.Cu) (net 8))
 (segment (start 69.735746 64.197792) (end 70.036066 64.498112) (width 0.2032) (layer F.Cu) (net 8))
 (segment (start 70.036066 64.498112) (end 70.362544 64.498112) (width 0.2032) (layer F.Cu) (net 8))
 (segment (start 70.362544 64.498112) (end 72.832208 66.967776) (width 0.2032) (layer F.Cu) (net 8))
 (segment (start 72.832208 66.967776) (end 72.832208 67.284254) (width 0.2032) (layer F.Cu) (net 8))
 (segment (start 73.5 63) (end 74.635 63) (width 0.2032) (layer B.Cu) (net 8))
 (segment (start 74.635 63) (end 75 62.635) (width 0.2032) (layer B.Cu) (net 8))
 (segment (start 75 62.635) (end 75 65.116462) (width 0.2032) (layer F.Cu) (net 8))
 (segment (start 75 65.116462) (end 72.832208 67.284254) (width 0.2032) (layer F.Cu) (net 8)))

